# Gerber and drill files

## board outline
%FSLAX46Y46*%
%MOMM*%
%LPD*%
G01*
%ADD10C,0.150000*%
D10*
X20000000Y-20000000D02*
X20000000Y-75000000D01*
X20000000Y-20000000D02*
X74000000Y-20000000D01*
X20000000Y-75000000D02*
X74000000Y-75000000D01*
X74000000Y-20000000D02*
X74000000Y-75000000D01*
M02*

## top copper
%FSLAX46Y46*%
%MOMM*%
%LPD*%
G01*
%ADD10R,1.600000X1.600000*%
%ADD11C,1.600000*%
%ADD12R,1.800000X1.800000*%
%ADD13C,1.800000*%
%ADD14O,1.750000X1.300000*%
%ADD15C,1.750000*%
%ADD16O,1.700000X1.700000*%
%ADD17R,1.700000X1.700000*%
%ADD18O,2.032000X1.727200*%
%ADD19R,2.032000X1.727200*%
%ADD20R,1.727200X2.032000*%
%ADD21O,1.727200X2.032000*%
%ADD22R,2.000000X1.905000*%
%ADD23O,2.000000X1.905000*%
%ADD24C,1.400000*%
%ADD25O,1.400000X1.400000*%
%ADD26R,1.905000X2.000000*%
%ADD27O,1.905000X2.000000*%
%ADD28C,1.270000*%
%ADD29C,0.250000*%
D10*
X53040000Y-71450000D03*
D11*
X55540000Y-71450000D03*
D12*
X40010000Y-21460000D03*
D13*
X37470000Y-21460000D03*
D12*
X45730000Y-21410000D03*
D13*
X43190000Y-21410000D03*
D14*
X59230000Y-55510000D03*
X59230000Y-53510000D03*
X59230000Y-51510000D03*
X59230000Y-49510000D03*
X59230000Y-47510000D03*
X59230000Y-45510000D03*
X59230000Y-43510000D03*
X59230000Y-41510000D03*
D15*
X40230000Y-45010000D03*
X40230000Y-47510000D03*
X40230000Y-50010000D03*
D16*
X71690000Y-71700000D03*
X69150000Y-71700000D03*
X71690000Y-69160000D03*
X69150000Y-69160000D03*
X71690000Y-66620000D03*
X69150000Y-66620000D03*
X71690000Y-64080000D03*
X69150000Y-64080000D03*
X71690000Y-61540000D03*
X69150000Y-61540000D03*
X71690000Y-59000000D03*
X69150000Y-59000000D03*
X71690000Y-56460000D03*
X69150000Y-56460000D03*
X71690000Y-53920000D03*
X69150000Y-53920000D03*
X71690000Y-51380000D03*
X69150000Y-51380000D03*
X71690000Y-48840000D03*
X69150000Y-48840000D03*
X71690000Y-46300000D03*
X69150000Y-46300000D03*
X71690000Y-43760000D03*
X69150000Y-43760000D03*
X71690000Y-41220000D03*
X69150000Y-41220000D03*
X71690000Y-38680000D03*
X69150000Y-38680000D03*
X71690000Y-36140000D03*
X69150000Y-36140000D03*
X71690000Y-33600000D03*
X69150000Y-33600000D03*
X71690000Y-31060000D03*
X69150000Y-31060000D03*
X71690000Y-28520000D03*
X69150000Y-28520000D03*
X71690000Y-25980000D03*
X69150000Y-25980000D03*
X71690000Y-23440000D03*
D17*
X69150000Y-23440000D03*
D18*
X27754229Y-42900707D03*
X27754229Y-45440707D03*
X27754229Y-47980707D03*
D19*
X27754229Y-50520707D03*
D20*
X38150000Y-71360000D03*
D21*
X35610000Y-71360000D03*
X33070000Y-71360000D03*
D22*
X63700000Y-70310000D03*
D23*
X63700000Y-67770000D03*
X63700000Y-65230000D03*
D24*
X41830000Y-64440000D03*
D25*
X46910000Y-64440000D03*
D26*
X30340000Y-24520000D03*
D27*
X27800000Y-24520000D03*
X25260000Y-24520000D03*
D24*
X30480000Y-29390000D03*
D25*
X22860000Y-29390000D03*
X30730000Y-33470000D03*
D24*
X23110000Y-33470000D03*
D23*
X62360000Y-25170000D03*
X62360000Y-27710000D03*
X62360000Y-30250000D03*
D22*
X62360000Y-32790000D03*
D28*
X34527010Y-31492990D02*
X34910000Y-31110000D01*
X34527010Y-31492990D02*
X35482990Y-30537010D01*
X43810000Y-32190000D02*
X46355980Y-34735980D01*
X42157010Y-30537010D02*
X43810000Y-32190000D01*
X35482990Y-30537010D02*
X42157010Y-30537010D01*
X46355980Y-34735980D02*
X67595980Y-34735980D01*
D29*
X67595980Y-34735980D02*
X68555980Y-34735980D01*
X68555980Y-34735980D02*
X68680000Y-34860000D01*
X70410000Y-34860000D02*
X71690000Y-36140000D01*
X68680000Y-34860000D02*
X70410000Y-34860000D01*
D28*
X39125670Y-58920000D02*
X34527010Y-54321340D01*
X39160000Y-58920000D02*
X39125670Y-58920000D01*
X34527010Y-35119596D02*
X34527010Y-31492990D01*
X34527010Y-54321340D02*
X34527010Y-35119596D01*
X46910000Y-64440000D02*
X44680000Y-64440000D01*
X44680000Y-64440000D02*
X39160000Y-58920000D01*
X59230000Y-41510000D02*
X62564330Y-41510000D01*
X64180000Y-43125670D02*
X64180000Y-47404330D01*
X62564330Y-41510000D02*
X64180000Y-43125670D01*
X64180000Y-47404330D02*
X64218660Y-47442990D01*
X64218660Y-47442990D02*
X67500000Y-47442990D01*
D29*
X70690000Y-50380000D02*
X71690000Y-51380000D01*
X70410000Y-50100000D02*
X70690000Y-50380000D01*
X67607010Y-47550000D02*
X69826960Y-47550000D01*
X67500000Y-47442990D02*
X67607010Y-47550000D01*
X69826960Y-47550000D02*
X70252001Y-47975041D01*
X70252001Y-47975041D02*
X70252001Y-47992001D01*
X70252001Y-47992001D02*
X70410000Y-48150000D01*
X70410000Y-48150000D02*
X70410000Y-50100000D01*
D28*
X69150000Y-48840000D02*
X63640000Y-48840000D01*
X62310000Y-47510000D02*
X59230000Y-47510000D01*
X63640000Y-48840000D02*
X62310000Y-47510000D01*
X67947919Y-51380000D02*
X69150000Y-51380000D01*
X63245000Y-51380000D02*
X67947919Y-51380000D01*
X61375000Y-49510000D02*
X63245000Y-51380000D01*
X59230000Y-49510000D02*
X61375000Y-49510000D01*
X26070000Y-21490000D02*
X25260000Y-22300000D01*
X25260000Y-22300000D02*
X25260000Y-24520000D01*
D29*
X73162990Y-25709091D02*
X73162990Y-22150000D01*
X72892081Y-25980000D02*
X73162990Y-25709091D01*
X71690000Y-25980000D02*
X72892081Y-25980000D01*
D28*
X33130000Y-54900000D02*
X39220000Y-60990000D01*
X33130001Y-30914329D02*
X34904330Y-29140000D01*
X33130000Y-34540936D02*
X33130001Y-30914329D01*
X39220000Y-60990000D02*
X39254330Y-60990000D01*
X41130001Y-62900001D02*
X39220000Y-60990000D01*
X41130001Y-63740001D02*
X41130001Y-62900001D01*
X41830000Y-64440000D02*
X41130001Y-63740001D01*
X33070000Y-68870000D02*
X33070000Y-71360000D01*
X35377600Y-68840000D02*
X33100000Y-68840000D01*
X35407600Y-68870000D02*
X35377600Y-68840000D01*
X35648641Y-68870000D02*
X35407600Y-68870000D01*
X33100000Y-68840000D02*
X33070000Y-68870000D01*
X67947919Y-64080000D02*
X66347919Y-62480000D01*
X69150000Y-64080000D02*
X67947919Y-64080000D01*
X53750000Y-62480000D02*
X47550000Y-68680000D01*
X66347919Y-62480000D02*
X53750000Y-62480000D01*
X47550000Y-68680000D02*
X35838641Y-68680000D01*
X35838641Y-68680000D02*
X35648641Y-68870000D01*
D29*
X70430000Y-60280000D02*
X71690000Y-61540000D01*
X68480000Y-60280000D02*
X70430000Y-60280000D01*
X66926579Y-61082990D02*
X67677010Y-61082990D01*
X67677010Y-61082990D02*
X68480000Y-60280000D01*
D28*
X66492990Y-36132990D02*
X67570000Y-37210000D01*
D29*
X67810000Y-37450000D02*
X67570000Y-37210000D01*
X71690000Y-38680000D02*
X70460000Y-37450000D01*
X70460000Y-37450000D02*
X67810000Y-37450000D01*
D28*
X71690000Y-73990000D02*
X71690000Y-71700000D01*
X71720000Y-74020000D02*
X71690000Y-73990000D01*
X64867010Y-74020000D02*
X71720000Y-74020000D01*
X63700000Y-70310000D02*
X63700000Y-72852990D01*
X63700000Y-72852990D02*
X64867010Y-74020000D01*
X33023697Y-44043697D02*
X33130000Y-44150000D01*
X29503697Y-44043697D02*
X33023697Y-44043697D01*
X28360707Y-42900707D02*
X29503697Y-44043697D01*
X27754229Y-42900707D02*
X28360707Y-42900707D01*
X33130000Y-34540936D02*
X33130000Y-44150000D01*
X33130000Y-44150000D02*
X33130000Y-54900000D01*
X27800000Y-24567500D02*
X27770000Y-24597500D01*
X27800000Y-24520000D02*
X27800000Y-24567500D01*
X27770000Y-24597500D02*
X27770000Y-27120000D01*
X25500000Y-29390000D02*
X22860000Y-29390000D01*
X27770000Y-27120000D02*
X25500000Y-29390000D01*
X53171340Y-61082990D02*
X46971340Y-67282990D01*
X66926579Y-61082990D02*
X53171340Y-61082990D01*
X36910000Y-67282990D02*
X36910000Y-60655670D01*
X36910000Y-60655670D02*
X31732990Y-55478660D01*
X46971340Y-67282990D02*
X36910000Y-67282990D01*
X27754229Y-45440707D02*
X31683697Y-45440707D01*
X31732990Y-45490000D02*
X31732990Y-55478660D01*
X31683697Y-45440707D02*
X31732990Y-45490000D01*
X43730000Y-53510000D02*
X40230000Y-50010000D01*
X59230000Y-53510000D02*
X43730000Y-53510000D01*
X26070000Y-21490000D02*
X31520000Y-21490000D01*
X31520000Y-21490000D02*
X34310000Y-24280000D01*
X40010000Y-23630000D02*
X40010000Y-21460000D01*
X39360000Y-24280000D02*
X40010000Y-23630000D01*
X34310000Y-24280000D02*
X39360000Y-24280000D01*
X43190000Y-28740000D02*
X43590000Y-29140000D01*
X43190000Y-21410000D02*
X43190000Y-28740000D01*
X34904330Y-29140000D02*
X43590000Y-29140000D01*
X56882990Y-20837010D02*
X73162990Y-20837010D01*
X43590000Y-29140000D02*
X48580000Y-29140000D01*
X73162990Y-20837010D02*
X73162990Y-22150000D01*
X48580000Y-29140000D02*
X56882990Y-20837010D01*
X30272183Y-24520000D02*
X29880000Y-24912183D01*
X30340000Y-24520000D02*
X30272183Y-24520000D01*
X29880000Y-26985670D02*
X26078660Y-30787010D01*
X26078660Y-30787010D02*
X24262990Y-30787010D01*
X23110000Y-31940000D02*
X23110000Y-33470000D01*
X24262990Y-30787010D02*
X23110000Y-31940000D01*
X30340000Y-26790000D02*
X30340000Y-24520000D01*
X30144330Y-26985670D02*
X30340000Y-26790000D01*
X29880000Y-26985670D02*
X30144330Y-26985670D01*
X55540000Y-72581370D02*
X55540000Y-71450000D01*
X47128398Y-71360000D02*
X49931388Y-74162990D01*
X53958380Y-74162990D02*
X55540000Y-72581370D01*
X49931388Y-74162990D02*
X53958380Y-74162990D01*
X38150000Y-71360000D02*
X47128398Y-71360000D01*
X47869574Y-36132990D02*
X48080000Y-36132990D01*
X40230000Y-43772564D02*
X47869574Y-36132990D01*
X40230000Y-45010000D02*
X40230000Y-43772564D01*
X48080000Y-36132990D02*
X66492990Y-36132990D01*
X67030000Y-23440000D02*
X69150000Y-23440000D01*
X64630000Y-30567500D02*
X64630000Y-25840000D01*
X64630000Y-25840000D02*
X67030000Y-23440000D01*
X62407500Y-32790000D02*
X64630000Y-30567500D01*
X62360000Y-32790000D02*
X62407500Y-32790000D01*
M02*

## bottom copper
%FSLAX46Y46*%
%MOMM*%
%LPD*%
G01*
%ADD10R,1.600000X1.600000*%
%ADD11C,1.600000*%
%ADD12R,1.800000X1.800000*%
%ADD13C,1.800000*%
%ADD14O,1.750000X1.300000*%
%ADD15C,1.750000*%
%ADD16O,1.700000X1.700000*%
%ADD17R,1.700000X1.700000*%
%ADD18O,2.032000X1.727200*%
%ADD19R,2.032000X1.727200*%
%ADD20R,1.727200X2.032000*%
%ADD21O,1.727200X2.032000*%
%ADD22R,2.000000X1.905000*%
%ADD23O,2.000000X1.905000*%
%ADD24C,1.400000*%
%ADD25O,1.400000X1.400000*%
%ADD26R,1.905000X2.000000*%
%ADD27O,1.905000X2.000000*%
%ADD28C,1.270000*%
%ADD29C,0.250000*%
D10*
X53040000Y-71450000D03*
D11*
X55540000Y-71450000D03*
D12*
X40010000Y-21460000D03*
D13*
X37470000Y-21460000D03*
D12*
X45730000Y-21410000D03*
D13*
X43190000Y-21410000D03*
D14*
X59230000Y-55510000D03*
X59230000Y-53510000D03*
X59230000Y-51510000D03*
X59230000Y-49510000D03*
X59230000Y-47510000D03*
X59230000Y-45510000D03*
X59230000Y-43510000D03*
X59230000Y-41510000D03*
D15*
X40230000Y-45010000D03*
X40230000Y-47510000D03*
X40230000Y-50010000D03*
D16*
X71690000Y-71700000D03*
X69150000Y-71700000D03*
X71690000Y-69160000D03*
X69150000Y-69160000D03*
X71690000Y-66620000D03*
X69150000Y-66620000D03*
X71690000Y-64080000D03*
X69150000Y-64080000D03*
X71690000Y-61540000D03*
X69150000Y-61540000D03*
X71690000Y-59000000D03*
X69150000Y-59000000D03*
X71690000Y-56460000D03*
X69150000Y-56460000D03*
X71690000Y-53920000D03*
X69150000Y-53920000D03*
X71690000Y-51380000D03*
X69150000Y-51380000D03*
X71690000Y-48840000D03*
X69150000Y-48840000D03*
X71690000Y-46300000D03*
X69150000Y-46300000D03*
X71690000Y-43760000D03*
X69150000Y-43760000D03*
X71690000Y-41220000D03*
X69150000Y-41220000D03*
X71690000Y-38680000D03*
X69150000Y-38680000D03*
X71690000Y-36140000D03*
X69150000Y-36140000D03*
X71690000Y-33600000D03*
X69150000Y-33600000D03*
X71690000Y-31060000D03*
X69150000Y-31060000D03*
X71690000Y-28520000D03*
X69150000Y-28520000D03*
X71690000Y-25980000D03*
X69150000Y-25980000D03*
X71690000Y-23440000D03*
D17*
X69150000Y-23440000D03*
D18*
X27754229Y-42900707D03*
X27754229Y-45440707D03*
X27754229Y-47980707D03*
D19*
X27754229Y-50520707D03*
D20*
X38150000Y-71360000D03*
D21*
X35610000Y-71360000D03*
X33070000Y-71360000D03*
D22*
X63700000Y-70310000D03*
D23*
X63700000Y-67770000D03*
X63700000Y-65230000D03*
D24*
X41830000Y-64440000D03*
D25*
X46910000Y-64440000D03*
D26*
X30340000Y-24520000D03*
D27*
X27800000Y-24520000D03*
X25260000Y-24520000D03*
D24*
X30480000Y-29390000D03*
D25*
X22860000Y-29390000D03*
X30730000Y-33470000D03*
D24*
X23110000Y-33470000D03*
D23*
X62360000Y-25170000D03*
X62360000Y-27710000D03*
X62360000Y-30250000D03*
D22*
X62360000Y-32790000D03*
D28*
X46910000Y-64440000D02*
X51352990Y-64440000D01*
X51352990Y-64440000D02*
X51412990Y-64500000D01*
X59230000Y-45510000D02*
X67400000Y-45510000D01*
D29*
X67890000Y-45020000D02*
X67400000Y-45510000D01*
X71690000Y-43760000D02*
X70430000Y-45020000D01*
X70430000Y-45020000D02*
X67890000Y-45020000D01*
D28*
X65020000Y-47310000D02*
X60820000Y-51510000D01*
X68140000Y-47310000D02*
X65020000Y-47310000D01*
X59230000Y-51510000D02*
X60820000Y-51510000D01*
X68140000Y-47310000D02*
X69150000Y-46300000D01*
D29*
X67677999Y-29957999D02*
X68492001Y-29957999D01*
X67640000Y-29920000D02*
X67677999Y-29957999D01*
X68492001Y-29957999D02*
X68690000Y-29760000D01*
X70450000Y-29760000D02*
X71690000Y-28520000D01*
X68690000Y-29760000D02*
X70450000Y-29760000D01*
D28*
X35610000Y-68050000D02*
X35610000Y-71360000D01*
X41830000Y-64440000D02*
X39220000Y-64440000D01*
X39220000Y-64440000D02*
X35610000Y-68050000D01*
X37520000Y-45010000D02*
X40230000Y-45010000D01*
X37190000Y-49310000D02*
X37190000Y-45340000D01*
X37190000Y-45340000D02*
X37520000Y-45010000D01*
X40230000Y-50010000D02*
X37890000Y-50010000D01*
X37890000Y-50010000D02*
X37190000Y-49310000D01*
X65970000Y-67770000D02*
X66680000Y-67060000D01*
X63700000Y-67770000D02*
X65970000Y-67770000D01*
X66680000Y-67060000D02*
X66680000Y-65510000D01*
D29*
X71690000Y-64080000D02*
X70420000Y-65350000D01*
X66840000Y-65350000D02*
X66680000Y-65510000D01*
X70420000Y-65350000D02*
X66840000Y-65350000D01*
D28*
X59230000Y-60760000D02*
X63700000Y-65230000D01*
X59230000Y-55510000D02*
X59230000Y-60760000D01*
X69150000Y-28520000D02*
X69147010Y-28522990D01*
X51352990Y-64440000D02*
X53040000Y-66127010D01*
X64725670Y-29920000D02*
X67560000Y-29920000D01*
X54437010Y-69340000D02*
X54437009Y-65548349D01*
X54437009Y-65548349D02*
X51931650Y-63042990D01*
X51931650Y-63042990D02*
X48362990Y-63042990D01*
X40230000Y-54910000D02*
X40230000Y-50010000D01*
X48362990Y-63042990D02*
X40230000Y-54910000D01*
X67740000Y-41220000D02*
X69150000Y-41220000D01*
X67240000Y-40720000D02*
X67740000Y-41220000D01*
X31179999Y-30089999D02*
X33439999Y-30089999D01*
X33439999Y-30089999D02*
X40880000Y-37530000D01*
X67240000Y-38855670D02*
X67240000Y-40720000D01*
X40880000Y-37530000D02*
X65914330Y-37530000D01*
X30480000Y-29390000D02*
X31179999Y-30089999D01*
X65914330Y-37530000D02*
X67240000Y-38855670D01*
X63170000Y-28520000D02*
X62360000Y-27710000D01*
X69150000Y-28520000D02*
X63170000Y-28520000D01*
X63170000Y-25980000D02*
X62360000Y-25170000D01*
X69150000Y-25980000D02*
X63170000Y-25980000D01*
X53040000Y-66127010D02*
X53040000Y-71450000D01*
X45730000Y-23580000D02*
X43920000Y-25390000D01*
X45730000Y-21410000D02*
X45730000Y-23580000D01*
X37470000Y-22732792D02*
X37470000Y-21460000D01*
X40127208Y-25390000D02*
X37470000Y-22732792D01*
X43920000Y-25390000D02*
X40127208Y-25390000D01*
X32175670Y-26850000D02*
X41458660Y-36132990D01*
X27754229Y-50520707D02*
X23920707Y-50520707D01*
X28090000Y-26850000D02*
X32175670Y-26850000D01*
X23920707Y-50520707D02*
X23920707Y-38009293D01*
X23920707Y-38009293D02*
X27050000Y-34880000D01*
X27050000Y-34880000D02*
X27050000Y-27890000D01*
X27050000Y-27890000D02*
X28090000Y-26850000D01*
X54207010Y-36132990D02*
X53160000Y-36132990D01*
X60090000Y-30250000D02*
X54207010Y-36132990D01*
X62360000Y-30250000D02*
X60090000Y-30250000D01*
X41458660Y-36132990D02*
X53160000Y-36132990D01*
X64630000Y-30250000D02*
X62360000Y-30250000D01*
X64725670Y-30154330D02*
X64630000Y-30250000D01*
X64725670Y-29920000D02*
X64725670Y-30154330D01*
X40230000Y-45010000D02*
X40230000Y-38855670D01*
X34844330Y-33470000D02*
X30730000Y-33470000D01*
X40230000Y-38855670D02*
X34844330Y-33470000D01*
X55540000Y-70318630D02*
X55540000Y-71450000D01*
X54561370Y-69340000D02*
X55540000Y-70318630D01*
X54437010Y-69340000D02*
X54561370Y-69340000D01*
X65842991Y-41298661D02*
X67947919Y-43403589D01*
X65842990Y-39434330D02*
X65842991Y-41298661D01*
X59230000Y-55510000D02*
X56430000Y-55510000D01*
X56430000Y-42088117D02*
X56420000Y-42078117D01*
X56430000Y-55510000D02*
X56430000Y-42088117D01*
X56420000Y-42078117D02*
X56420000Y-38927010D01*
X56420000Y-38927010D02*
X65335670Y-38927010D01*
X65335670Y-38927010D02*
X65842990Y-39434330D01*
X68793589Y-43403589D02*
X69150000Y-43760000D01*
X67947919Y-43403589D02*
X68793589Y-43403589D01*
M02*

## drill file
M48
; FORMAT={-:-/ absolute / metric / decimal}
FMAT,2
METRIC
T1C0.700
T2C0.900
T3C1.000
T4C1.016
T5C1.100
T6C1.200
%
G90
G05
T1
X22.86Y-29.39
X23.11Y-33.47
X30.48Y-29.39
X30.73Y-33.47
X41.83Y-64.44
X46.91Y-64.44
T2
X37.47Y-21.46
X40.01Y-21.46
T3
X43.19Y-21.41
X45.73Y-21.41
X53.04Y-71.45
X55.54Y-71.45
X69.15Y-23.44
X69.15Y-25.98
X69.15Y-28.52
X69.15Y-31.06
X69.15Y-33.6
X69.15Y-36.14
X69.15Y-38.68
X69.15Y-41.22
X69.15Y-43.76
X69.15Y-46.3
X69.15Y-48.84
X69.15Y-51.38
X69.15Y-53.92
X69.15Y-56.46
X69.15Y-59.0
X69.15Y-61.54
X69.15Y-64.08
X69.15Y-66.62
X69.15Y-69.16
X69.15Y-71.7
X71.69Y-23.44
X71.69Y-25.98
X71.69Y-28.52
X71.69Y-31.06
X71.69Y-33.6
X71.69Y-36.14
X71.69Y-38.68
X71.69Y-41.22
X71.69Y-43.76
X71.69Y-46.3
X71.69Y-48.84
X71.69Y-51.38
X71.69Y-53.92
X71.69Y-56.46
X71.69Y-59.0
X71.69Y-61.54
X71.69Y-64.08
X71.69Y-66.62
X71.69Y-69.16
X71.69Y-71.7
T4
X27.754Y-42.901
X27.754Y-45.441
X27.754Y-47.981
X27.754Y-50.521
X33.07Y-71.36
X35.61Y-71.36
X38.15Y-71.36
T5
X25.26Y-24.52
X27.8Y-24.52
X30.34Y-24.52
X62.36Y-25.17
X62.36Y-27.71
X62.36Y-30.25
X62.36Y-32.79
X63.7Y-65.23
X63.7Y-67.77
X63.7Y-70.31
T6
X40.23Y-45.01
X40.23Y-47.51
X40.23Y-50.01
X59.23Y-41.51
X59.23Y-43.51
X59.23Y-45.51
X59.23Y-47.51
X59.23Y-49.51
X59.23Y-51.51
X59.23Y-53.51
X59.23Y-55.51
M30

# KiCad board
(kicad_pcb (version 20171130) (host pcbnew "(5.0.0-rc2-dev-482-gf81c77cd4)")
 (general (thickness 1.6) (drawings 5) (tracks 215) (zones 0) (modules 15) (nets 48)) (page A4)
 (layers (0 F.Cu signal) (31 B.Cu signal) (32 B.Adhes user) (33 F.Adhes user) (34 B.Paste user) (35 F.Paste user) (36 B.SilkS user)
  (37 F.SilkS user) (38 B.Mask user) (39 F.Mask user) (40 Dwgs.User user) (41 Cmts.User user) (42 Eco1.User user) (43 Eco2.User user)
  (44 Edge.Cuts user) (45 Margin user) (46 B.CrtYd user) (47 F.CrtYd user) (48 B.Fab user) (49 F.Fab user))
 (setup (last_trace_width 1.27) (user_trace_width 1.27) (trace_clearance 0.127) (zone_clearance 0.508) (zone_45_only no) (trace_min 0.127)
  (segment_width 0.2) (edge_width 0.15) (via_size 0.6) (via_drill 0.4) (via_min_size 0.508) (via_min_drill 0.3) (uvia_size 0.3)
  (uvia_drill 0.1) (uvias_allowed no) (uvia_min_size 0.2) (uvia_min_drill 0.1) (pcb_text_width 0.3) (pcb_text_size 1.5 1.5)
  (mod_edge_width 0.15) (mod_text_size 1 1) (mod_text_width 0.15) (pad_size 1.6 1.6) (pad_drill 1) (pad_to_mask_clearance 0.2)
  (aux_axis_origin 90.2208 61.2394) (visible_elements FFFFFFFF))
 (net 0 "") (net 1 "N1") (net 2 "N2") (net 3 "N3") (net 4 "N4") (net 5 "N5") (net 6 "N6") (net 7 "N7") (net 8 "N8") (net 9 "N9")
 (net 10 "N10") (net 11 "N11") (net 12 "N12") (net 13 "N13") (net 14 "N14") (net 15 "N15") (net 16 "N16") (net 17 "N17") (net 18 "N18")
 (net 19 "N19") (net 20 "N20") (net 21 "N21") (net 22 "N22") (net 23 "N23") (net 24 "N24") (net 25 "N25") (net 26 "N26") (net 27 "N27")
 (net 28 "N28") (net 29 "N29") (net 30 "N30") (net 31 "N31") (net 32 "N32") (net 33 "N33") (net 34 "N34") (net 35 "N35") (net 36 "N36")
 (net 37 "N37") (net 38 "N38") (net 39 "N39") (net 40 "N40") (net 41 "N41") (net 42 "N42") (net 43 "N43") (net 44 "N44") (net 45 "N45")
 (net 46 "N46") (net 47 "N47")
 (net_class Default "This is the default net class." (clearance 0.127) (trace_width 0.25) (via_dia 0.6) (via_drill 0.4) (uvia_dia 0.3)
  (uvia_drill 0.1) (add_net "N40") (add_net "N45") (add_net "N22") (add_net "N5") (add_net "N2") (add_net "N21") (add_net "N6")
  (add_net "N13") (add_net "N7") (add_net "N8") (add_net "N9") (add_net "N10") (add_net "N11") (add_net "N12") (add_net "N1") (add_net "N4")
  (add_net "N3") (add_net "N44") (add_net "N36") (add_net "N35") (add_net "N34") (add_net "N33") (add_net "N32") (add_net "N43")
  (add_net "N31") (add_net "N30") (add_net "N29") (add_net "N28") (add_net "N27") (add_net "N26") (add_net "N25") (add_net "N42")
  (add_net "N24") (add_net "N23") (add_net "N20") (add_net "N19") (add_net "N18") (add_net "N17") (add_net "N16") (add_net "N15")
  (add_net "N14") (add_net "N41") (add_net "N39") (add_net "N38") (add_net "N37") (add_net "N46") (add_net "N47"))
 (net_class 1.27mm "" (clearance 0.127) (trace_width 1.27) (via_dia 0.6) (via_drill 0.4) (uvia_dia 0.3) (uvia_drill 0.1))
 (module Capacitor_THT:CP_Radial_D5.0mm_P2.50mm (layer F.Cu) (at 53.04 71.45)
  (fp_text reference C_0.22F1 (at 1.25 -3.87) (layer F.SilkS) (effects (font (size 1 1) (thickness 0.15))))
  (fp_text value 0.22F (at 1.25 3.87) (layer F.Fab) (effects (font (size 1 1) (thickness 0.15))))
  (pad 1 thru_hole rect (at 0 0) (size 1.6 1.6) (drill 1) (layers *.Cu *.Mask) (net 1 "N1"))
  (pad 2 thru_hole circle (at 2.5 0) (size 1.6 1.6) (drill 1) (layers *.Cu *.Mask) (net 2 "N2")))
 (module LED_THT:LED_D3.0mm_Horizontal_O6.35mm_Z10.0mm (layer F.Cu) (at 40.01 21.46 180)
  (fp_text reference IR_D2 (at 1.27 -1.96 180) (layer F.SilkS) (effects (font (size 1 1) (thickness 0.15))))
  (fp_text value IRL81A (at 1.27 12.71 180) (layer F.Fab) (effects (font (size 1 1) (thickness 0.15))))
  (pad 1 thru_hole rect (at 0 0 180) (size 1.8 1.8) (drill 0.9) (layers *.Cu *.Mask) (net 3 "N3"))
  (pad 2 thru_hole circle (at 2.54 0 180) (size 1.8 1.8) (drill 0.9) (layers *.Cu *.Mask) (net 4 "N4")))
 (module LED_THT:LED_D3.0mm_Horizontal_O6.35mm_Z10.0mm (layer F.Cu) (at 45.73 21.41 180)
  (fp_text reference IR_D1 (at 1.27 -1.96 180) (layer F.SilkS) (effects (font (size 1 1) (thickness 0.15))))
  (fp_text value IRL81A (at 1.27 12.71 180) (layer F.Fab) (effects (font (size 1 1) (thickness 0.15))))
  (pad 1 thru_hole rect (at 0 0 180) (size 1.8 1.8) (drill 1) (layers *.Cu *.Mask) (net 4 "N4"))
  (pad 2 thru_hole circle (at 2.54 0 180) (size 1.8 1.8) (drill 1) (layers *.Cu *.Mask) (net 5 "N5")))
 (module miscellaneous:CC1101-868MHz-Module (layer F.Cu) (at 49.73 48.51 180)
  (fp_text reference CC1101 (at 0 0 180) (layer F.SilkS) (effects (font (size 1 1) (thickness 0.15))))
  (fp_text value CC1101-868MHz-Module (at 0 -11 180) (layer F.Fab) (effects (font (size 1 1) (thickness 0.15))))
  (pad 1 thru_hole oval (at -9.5 -7 180) (size 1.75 1.3) (drill 1.2) (layers *.Cu *.Mask) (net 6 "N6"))
  (pad 2 thru_hole oval (at -9.5 -5 180) (size 1.75 1.3) (drill 1.2) (layers *.Cu *.Mask) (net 2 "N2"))
  (pad 3 thru_hole oval (at -9.5 -3 180) (size 1.75 1.3) (drill 1.2) (layers *.Cu *.Mask) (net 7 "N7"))
  (pad 4 thru_hole oval (at -9.5 -1 180) (size 1.75 1.3) (drill 1.2) (layers *.Cu *.Mask) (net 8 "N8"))
  (pad 5 thru_hole oval (at -9.5 1 180) (size 1.75 1.3) (drill 1.2) (layers *.Cu *.Mask) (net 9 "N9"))
  (pad 6 thru_hole oval (at -9.5 3 180) (size 1.75 1.3) (drill 1.2) (layers *.Cu *.Mask) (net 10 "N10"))
  (pad 7 thru_hole oval (at -9.5 5 180) (size 1.75 1.3) (drill 1.2) (layers *.Cu *.Mask) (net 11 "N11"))
  (pad 8 thru_hole oval (at -9.5 7 180) (size 1.75 1.3) (drill 1.2) (layers *.Cu *.Mask) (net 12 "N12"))
  (pad 9 thru_hole circle (at 9.5 3.5 180) (size 1.75 1.75) (drill 1.2) (layers *.Cu *.Mask) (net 2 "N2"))
  (pad 10 thru_hole circle (at 9.5 1 180) (size 1.75 1.75) (drill 1.2) (layers *.Cu *.Mask) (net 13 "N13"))
  (pad 11 thru_hole circle (at 9.5 -1.5 180) (size 1.75 1.75) (drill 1.2) (layers *.Cu *.Mask) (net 2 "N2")))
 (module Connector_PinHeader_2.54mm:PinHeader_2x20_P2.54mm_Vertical (layer F.Cu) (at 69.15 23.44)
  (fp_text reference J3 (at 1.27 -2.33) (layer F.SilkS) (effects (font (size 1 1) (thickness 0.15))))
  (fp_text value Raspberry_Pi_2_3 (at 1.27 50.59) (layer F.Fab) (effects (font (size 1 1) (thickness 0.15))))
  (pad 40 thru_hole oval (at 2.54 48.26) (size 1.7 1.7) (drill 1) (layers *.Cu *.Mask) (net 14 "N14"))
  (pad 39 thru_hole oval (at 0 48.26) (size 1.7 1.7) (drill 1) (layers *.Cu *.Mask) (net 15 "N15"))
  (pad 38 thru_hole oval (at 2.54 45.72) (size 1.7 1.7) (drill 1) (layers *.Cu *.Mask) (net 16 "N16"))
  (pad 37 thru_hole oval (at 0 45.72) (size 1.7 1.7) (drill 1) (layers *.Cu *.Mask) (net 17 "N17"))
  (pad 36 thru_hole oval (at 2.54 43.18) (size 1.7 1.7) (drill 1) (layers *.Cu *.Mask) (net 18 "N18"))
  (pad 35 thru_hole oval (at 0 43.18) (size 1.7 1.7) (drill 1) (layers *.Cu *.Mask) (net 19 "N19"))
  (pad 34 thru_hole oval (at 2.54 40.64) (size 1.7 1.7) (drill 1) (layers *.Cu *.Mask) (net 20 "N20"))
  (pad 33 thru_hole oval (at 0 40.64) (size 1.7 1.7) (drill 1) (layers *.Cu *.Mask) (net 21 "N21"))
  (pad 32 thru_hole oval (at 2.54 38.1) (size 1.7 1.7) (drill 1) (layers *.Cu *.Mask) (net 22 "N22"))
  (pad 31 thru_hole oval (at 0 38.1) (size 1.7 1.7) (drill 1) (layers *.Cu *.Mask) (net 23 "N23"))
  (pad 30 thru_hole oval (at 2.54 35.56) (size 1.7 1.7) (drill 1) (layers *.Cu *.Mask) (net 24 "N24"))
  (pad 29 thru_hole oval (at 0 35.56) (size 1.7 1.7) (drill 1) (layers *.Cu *.Mask) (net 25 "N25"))
  (pad 28 thru_hole oval (at 2.54 33.02) (size 1.7 1.7) (drill 1) (layers *.Cu *.Mask) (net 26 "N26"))
  (pad 27 thru_hole oval (at 0 33.02) (size 1.7 1.7) (drill 1) (layers *.Cu *.Mask) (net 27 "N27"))
  (pad 26 thru_hole oval (at 2.54 30.48) (size 1.7 1.7) (drill 1) (layers *.Cu *.Mask) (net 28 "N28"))
  (pad 25 thru_hole oval (at 0 30.48) (size 1.7 1.7) (drill 1) (layers *.Cu *.Mask) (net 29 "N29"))
  (pad 24 thru_hole oval (at 2.54 27.94) (size 1.7 1.7) (drill 1) (layers *.Cu *.Mask) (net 12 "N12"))
  (pad 23 thru_hole oval (at 0 27.94) (size 1.7 1.7) (drill 1) (layers *.Cu *.Mask) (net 8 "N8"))
  (pad 22 thru_hole oval (at 2.54 25.4) (size 1.7 1.7) (drill 1) (layers *.Cu *.Mask) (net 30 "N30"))
  (pad 21 thru_hole oval (at 0 25.4) (size 1.7 1.7) (drill 1) (layers *.Cu *.Mask) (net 9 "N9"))
  (pad 20 thru_hole oval (at 2.54 22.86) (size 1.7 1.7) (drill 1) (layers *.Cu *.Mask) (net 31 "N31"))
  (pad 19 thru_hole oval (at 0 22.86) (size 1.7 1.7) (drill 1) (layers *.Cu *.Mask) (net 7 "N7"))
  (pad 18 thru_hole oval (at 2.54 20.32) (size 1.7 1.7) (drill 1) (layers *.Cu *.Mask) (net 10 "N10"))
  (pad 17 thru_hole oval (at 0 20.32) (size 1.7 1.7) (drill 1) (layers *.Cu *.Mask) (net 6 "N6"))
  (pad 16 thru_hole oval (at 2.54 17.78) (size 1.7 1.7) (drill 1) (layers *.Cu *.Mask) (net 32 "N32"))
  (pad 15 thru_hole oval (at 0 17.78) (size 1.7 1.7) (drill 1) (layers *.Cu *.Mask) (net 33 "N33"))
  (pad 14 thru_hole oval (at 2.54 15.24) (size 1.7 1.7) (drill 1) (layers *.Cu *.Mask) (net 2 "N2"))
  (pad 13 thru_hole oval (at 0 15.24) (size 1.7 1.7) (drill 1) (layers *.Cu *.Mask) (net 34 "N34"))
  (pad 12 thru_hole oval (at 2.54 12.7) (size 1.7 1.7) (drill 1) (layers *.Cu *.Mask) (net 1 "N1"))
  (pad 11 thru_hole oval (at 0 12.7) (size 1.7 1.7) (drill 1) (layers *.Cu *.Mask) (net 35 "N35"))
  (pad 10 thru_hole oval (at 2.54 10.16) (size 1.7 1.7) (drill 1) (layers *.Cu *.Mask) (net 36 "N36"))
  (pad 9 thru_hole oval (at 0 10.16) (size 1.7 1.7) (drill 1) (layers *.Cu *.Mask) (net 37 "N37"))
  (pad 8 thru_hole oval (at 2.54 7.62) (size 1.7 1.7) (drill 1) (layers *.Cu *.Mask) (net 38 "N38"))
  (pad 7 thru_hole oval (at 0 7.62) (size 1.7 1.7) (drill 1) (layers *.Cu *.Mask) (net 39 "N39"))
  (pad 6 thru_hole oval (at 2.54 5.08) (size 1.7 1.7) (drill 1) (layers *.Cu *.Mask) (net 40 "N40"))
  (pad 5 thru_hole oval (at 0 5.08) (size 1.7 1.7) (drill 1) (layers *.Cu *.Mask) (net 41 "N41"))
  (pad 4 thru_hole oval (at 2.54 2.54) (size 1.7 1.7) (drill 1) (layers *.Cu *.Mask) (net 5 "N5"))
  (pad 3 thru_hole oval (at 0 2.54) (size 1.7 1.7) (drill 1) (layers *.Cu *.Mask) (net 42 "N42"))
  (pad 2 thru_hole oval (at 2.54 0) (size 1.7 1.7) (drill 1) (layers *.Cu *.Mask) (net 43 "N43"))
  (pad 1 thru_hole rect (at 0 0) (size 1.7 1.7) (drill 1) (layers *.Cu *.Mask) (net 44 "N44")))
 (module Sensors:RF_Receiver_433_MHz (layer F.Cu) (at 27.73 45.46 90)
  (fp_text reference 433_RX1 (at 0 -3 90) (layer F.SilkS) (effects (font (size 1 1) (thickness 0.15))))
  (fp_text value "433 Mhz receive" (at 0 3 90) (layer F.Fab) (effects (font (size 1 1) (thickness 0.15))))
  (pad 4 thru_hole oval (at 2.559293 0.024229 180) (size 2.032 1.7272) (drill 1.016) (layers *.Cu *.Mask F.SilkS) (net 5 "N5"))
  (pad 3 thru_hole oval (at 0.019293 0.024229 180) (size 2.032 1.7272) (drill 1.016) (layers *.Cu *.Mask F.SilkS) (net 22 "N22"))
  (pad 2 thru_hole oval (at -2.520707 0.024229 180) (size 2.032 1.7272) (drill 1.016) (layers *.Cu *.Mask F.SilkS) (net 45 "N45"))
  (pad 1 thru_hole rect (at -5.060707 0.024229 180) (size 2.032 1.7272) (drill 1.016) (layers *.Cu *.Mask F.SilkS) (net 40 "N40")))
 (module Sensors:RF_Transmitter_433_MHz (layer F.Cu) (at 35.61 71.36 180)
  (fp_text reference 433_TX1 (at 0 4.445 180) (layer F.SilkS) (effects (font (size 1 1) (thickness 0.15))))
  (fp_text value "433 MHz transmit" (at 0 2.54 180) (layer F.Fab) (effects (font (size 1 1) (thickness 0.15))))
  (pad 1 thru_hole rect (at -2.54 0 270) (size 2.032 1.7272) (drill 1.016) (layers *.Cu *.Mask F.SilkS) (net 2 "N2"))
  (pad 2 thru_hole oval (at 0 0 270) (size 2.032 1.7272) (drill 1.016) (layers *.Cu *.Mask F.SilkS) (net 5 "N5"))
  (pad 3 thru_hole oval (at 2.54 0 270) (size 2.032 1.7272) (drill 1.016) (layers *.Cu *.Mask F.SilkS) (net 21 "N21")))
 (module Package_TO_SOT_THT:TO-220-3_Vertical (layer F.Cu) (at 63.7 70.31 90)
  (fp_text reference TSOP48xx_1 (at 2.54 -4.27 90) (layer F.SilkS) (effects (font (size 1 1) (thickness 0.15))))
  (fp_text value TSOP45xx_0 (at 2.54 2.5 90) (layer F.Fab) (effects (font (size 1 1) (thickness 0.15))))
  (pad 1 thru_hole rect (at 0 0 90) (size 1.905 2) (drill 1.1) (layers *.Cu *.Mask) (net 14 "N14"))
  (pad 2 thru_hole oval (at 2.54 0 90) (size 1.905 2) (drill 1.1) (layers *.Cu *.Mask) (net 20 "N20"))
  (pad 3 thru_hole oval (at 5.08 0 90) (size 1.905 2) (drill 1.1) (layers *.Cu *.Mask) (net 6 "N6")))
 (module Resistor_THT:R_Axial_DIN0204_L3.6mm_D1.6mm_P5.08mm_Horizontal (layer F.Cu) (at 41.83 64.44)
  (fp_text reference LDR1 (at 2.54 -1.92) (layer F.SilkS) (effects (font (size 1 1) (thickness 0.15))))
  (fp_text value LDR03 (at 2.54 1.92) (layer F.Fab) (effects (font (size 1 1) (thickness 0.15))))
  (pad 1 thru_hole circle (at 0 0) (size 1.4 1.4) (drill 0.7) (layers *.Cu *.Mask) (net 5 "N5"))
  (pad 2 thru_hole oval (at 5.08 0) (size 1.4 1.4) (drill 0.7) (layers *.Cu *.Mask) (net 1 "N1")))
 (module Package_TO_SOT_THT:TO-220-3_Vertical (layer F.Cu) (at 30.34 24.52 180)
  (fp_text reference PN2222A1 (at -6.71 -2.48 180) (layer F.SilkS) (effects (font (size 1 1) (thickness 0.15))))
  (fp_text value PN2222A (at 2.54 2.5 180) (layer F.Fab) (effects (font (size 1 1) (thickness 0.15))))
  (pad 1 thru_hole rect (at 0 0 180) (size 1.905 2) (drill 1.1) (layers *.Cu *.Mask) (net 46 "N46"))
  (pad 2 thru_hole oval (at 2.54 0 180) (size 1.905 2) (drill 1.1) (layers *.Cu *.Mask) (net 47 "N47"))
  (pad 3 thru_hole oval (at 5.08 0 180) (size 1.905 2) (drill 1.1) (layers *.Cu *.Mask) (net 3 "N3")))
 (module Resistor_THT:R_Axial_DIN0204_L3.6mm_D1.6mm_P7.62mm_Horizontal (layer F.Cu) (at 30.48 29.39 180)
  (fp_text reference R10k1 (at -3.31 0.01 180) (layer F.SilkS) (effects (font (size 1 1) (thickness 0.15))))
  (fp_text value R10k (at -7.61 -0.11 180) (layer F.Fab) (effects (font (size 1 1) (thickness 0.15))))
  (pad 1 thru_hole circle (at 0 0 180) (size 1.4 1.4) (drill 0.7) (layers *.Cu *.Mask) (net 33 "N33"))
  (pad 2 thru_hole oval (at 7.62 0 180) (size 1.4 1.4) (drill 0.7) (layers *.Cu *.Mask) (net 47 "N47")))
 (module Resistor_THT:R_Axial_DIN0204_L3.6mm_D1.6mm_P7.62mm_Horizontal (layer F.Cu) (at 23.11 33.47)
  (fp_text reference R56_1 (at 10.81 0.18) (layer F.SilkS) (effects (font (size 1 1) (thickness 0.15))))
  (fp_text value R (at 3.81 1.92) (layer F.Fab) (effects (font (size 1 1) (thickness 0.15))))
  (pad 2 thru_hole oval (at 7.62 0) (size 1.4 1.4) (drill 0.7) (layers *.Cu *.Mask) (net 2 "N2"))
  (pad 1 thru_hole circle (at 0 0) (size 1.4 1.4) (drill 0.7) (layers *.Cu *.Mask) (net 46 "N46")))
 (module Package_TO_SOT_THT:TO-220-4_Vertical (layer F.Cu) (at 62.36 32.79 90)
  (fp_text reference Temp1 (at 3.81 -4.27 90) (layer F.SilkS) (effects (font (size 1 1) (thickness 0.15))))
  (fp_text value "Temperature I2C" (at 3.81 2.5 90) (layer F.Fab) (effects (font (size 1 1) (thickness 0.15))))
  (pad 4 thru_hole oval (at 7.62 0 90) (size 1.905 2) (drill 1.1) (layers *.Cu *.Mask) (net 42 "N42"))
  (pad 3 thru_hole oval (at 5.08 0 90) (size 1.905 2) (drill 1.1) (layers *.Cu *.Mask) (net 41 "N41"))
  (pad 2 thru_hole oval (at 2.54 0 90) (size 1.905 2) (drill 1.1) (layers *.Cu *.Mask) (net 40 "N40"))
  (pad 1 thru_hole rect (at 0 0 90) (size 1.905 2) (drill 1.1) (layers *.Cu *.Mask) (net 44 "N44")))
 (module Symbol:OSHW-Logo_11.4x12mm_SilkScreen (layer F.Cu) (at 51.43 27.68)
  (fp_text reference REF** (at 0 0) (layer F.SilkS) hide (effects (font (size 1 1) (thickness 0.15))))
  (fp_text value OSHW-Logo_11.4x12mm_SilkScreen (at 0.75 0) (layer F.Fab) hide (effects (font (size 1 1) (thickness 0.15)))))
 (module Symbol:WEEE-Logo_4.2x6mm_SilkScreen (layer F.Cu) (at 22.62 71.55)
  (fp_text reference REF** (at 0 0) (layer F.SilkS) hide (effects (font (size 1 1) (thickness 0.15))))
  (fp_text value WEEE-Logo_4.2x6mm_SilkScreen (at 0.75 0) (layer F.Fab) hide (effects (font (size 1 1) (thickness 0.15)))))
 (gr_line (start 20 20) (end 20 75) (angle 90) (layer Edge.Cuts) (width 0.15))
 (gr_line (start 20 20) (end 74 20) (angle 90) (layer Edge.Cuts) (width 0.15))
 (gr_line (start 20 75) (end 74 75) (angle 90) (layer Edge.Cuts) (width 0.15))
 (gr_line (start 74 20) (end 74 75) (angle 90) (layer Edge.Cuts) (width 0.15))
 (segment (start 34.52701 31.49299) (end 34.91 31.11) (width 1.27) (layer F.Cu) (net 1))
 (segment (start 34.52701 31.49299) (end 35.48299 30.53701) (width 1.27) (layer F.Cu) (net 1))
 (segment (start 43.81 32.19) (end 46.35598 34.73598) (width 1.27) (layer F.Cu) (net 1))
 (segment (start 42.15701 30.53701) (end 43.81 32.19) (width 1.27) (layer F.Cu) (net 1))
 (segment (start 35.48299 30.53701) (end 42.15701 30.53701) (width 1.27) (layer F.Cu) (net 1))
 (segment (start 46.35598 34.73598) (end 67.59598 34.73598) (width 1.27) (layer F.Cu) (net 1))
 (segment (start 67.59598 34.73598) (end 68.55598 34.73598) (width 0.25) (layer F.Cu) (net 1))
 (segment (start 68.55598 34.73598) (end 68.68 34.86) (width 0.25) (layer F.Cu) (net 1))
 (segment (start 70.41 34.86) (end 71.69 36.14) (width 0.25) (layer F.Cu) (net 1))
 (segment (start 68.68 34.86) (end 70.41 34.86) (width 0.25) (layer F.Cu) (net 1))
 (segment (start 39.12567 58.92) (end 34.52701 54.32134) (width 1.27) (layer F.Cu) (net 1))
 (segment (start 39.16 58.92) (end 39.12567 58.92) (width 1.27) (layer F.Cu) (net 1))
 (segment (start 34.52701 35.119596) (end 34.52701 31.49299) (width 1.27) (layer F.Cu) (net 1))
 (segment (start 34.52701 54.32134) (end 34.52701 35.119596) (width 1.27) (layer F.Cu) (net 1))
 (segment (start 46.91 64.44) (end 44.68 64.44) (width 1.27) (layer F.Cu) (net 1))
 (segment (start 44.68 64.44) (end 39.16 58.92) (width 1.27) (layer F.Cu) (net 1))
 (segment (start 46.91 64.44) (end 51.35299 64.44) (width 1.27) (layer B.Cu) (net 1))
 (segment (start 51.35299 64.44) (end 51.41299 64.5) (width 1.27) (layer B.Cu) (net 1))
 (segment (start 59.23 41.51) (end 62.56433 41.51) (width 1.27) (layer F.Cu) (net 12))
 (segment (start 64.18 43.12567) (end 64.18 47.40433) (width 1.27) (layer F.Cu) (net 12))
 (segment (start 62.56433 41.51) (end 64.18 43.12567) (width 1.27) (layer F.Cu) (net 12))
 (segment (start 64.18 47.40433) (end 64.21866 47.44299) (width 1.27) (layer F.Cu) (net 12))
 (segment (start 64.21866 47.44299) (end 67.5 47.44299) (width 1.27) (layer F.Cu) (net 12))
 (segment (start 70.69 50.38) (end 71.69 51.38) (width 0.25) (layer F.Cu) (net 12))
 (segment (start 70.41 50.1) (end 70.69 50.38) (width 0.25) (layer F.Cu) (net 12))
 (segment (start 67.60701 47.55) (end 69.82696 47.55) (width 0.25) (layer F.Cu) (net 12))
 (segment (start 67.5 47.44299) (end 67.60701 47.55) (width 0.25) (layer F.Cu) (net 12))
 (segment (start 69.82696 47.55) (end 70.252001 47.975041) (width 0.25) (layer F.Cu) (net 12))
 (segment (start 70.252001 47.975041) (end 70.252001 47.992001) (width 0.25) (layer F.Cu) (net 12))
 (segment (start 70.252001 47.992001) (end 70.41 48.15) (width 0.25) (layer F.Cu) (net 12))
 (segment (start 70.41 48.15) (end 70.41 50.1) (width 0.25) (layer F.Cu) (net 12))
 (segment (start 59.23 45.51) (end 67.4 45.51) (width 1.27) (layer B.Cu) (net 10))
 (segment (start 67.89 45.02) (end 67.4 45.51) (width 0.25) (layer B.Cu) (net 10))
 (segment (start 71.69 43.76) (end 70.43 45.02) (width 0.25) (layer B.Cu) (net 10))
 (segment (start 70.43 45.02) (end 67.89 45.02) (width 0.25) (layer B.Cu) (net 10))
 (segment (start 69.15 48.84) (end 63.64 48.84) (width 1.27) (layer F.Cu) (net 9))
 (segment (start 62.31 47.51) (end 59.23 47.51) (width 1.27) (layer F.Cu) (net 9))
 (segment (start 63.64 48.84) (end 62.31 47.51) (width 1.27) (layer F.Cu) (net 9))
 (segment (start 67.947919 51.38) (end 69.15 51.38) (width 1.27) (layer F.Cu) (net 8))
 (segment (start 63.245 51.38) (end 67.947919 51.38) (width 1.27) (layer F.Cu) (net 8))
 (segment (start 61.375 49.51) (end 63.245 51.38) (width 1.27) (layer F.Cu) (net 8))
 (segment (start 59.23 49.51) (end 61.375 49.51) (width 1.27) (layer F.Cu) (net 8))
 (segment (start 65.02 47.31) (end 60.82 51.51) (width 1.27) (layer B.Cu) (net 7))
 (segment (start 68.14 47.31) (end 65.02 47.31) (width 1.27) (layer B.Cu) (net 7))
 (segment (start 59.23 51.51) (end 60.82 51.51) (width 1.27) (layer B.Cu) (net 7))
 (segment (start 68.14 47.31) (end 69.15 46.3) (width 1.27) (layer B.Cu) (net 7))
 (segment (start 26.07 21.49) (end 25.26 22.3) (width 1.27) (layer F.Cu) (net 3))
 (segment (start 25.26 22.3) (end 25.26 24.52) (width 1.27) (layer F.Cu) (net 3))
 (segment (start 67.677999 29.957999) (end 68.492001 29.957999) (width 0.25) (layer B.Cu) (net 40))
 (segment (start 67.64 29.92) (end 67.677999 29.957999) (width 0.25) (layer B.Cu) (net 40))
 (segment (start 68.492001 29.957999) (end 68.69 29.76) (width 0.25) (layer B.Cu) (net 40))
 (segment (start 70.45 29.76) (end 71.69 28.52) (width 0.25) (layer B.Cu) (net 40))
 (segment (start 68.69 29.76) (end 70.45 29.76) (width 0.25) (layer B.Cu) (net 40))
 (segment (start 73.16299 25.709091) (end 73.16299 22.15) (width 0.25) (layer F.Cu) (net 5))
 (segment (start 72.892081 25.98) (end 73.16299 25.709091) (width 0.25) (layer F.Cu) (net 5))
 (segment (start 71.69 25.98) (end 72.892081 25.98) (width 0.25) (layer F.Cu) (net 5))
 (segment (start 33.13 54.9) (end 39.22 60.99) (width 1.27) (layer F.Cu) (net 5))
 (segment (start 33.130001 30.914329) (end 34.90433 29.14) (width 1.27) (layer F.Cu) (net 5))
 (segment (start 33.13 34.540936) (end 33.130001 30.914329) (width 1.27) (layer F.Cu) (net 5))
 (segment (start 39.22 60.99) (end 39.25433 60.99) (width 1.27) (layer F.Cu) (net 5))
 (segment (start 41.130001 62.900001) (end 39.22 60.99) (width 1.27) (layer F.Cu) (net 5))
 (segment (start 41.130001 63.740001) (end 41.130001 62.900001) (width 1.27) (layer F.Cu) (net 5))
 (segment (start 41.83 64.44) (end 41.130001 63.740001) (width 1.27) (layer F.Cu) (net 5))
 (segment (start 35.61 68.05) (end 35.61 71.36) (width 1.27) (layer B.Cu) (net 5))
 (segment (start 41.83 64.44) (end 39.22 64.44) (width 1.27) (layer B.Cu) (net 5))
 (segment (start 39.22 64.44) (end 35.61 68.05) (width 1.27) (layer B.Cu) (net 5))
 (segment (start 33.07 68.87) (end 33.07 71.36) (width 1.27) (layer F.Cu) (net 21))
 (segment (start 35.3776 68.84) (end 33.1 68.84) (width 1.27) (layer F.Cu) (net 21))
 (segment (start 35.4076 68.87) (end 35.3776 68.84) (width 1.27) (layer F.Cu) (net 21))
 (segment (start 35.648641 68.87) (end 35.4076 68.87) (width 1.27) (layer F.Cu) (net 21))
 (segment (start 33.1 68.84) (end 33.07 68.87) (width 1.27) (layer F.Cu) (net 21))
 (segment (start 67.947919 64.08) (end 66.347919 62.48) (width 1.27) (layer F.Cu) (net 21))
 (segment (start 69.15 64.08) (end 67.947919 64.08) (width 1.27) (layer F.Cu) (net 21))
 (segment (start 53.75 62.48) (end 47.55 68.68) (width 1.27) (layer F.Cu) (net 21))
 (segment (start 66.347919 62.48) (end 53.75 62.48) (width 1.27) (layer F.Cu) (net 21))
 (segment (start 47.55 68.68) (end 35.838641 68.68) (width 1.27) (layer F.Cu) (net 21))
 (segment (start 35.838641 68.68) (end 35.648641 68.87) (width 1.27) (layer F.Cu) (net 21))
 (segment (start 70.43 60.28) (end 71.69 61.54) (width 0.25) (layer F.Cu) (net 22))
 (segment (start 68.48 60.28) (end 70.43 60.28) (width 0.25) (layer F.Cu) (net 22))
 (segment (start 66.926579 61.08299) (end 67.67701 61.08299) (width 0.25) (layer F.Cu) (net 22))
 (segment (start 67.67701 61.08299) (end 68.48 60.28) (width 0.25) (layer F.Cu) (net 22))
 (segment (start 66.49299 36.13299) (end 67.57 37.21) (width 1.27) (layer F.Cu) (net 2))
 (segment (start 67.81 37.45) (end 67.57 37.21) (width 0.25) (layer F.Cu) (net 2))
 (segment (start 71.69 38.68) (end 70.46 37.45) (width 0.25) (layer F.Cu) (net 2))
 (segment (start 70.46 37.45) (end 67.81 37.45) (width 0.25) (layer F.Cu) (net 2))
 (segment (start 37.52 45.01) (end 40.23 45.01) (width 1.27) (layer B.Cu) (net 2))
 (segment (start 37.19 49.31) (end 37.19 45.34) (width 1.27) (layer B.Cu) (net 2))
 (segment (start 37.19 45.34) (end 37.52 45.01) (width 1.27) (layer B.Cu) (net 2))
 (segment (start 40.23 50.01) (end 37.89 50.01) (width 1.27) (layer B.Cu) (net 2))
 (segment (start 37.89 50.01) (end 37.19 49.31) (width 1.27) (layer B.Cu) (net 2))
 (segment (start 71.69 73.99) (end 71.69 71.7) (width 1.27) (layer F.Cu) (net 14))
 (segment (start 71.72 74.02) (end 71.69 73.99) (width 1.27) (layer F.Cu) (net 14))
 (segment (start 64.86701 74.02) (end 71.72 74.02) (width 1.27) (layer F.Cu) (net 14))
 (segment (start 63.7 70.31) (end 63.7 72.85299) (width 1.27) (layer F.Cu) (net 14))
 (segment (start 63.7 72.85299) (end 64.86701 74.02) (width 1.27) (layer F.Cu) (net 14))
 (segment (start 65.97 67.77) (end 66.68 67.06) (width 1.27) (layer B.Cu) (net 20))
 (segment (start 63.7 67.77) (end 65.97 67.77) (width 1.27) (layer B.Cu) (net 20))
 (segment (start 66.68 67.06) (end 66.68 65.51) (width 1.27) (layer B.Cu) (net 20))
 (segment (start 71.69 64.08) (end 70.42 65.35) (width 0.25) (layer B.Cu) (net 20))
 (segment (start 66.84 65.35) (end 66.68 65.51) (width 0.25) (layer B.Cu) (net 20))
 (segment (start 70.42 65.35) (end 66.84 65.35) (width 0.25) (layer B.Cu) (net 20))
 (segment (start 59.23 60.76) (end 63.7 65.23) (width 1.27) (layer B.Cu) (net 6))
 (segment (start 59.23 55.51) (end 59.23 60.76) (width 1.27) (layer B.Cu) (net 6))
 (segment (start 69.15 28.52) (end 69.14701 28.52299) (width 1.27) (layer B.Cu) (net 41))
 (segment (start 51.35299 64.44) (end 53.04 66.12701) (width 1.27) (layer B.Cu) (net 1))
 (segment (start 64.72567 29.92) (end 67.56 29.92) (width 1.27) (layer B.Cu) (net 40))
 (segment (start 33.023697 44.043697) (end 33.13 44.15) (width 1.27) (layer F.Cu) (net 5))
 (segment (start 29.503697 44.043697) (end 33.023697 44.043697) (width 1.27) (layer F.Cu) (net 5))
 (segment (start 28.360707 42.900707) (end 29.503697 44.043697) (width 1.27) (layer F.Cu) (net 5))
 (segment (start 27.754229 42.900707) (end 28.360707 42.900707) (width 1.27) (layer F.Cu) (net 5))
 (segment (start 33.13 34.540936) (end 33.13 44.15) (width 1.27) (layer F.Cu) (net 5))
 (segment (start 33.13 44.15) (end 33.13 54.9) (width 1.27) (layer F.Cu) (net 5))
 (segment (start 27.8 24.5675) (end 27.77 24.5975) (width 1.27) (layer F.Cu) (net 47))
 (segment (start 27.8 24.52) (end 27.8 24.5675) (width 1.27) (layer F.Cu) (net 47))
 (segment (start 27.77 24.5975) (end 27.77 27.12) (width 1.27) (layer F.Cu) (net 47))
 (segment (start 25.5 29.39) (end 22.86 29.39) (width 1.27) (layer F.Cu) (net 47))
 (segment (start 27.77 27.12) (end 25.5 29.39) (width 1.27) (layer F.Cu) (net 47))
 (segment (start 53.17134 61.08299) (end 46.97134 67.28299) (width 1.27) (layer F.Cu) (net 22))
 (segment (start 66.926579 61.08299) (end 53.17134 61.08299) (width 1.27) (layer F.Cu) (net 22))
 (segment (start 36.91 67.28299) (end 36.91 60.65567) (width 1.27) (layer F.Cu) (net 22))
 (segment (start 36.91 60.65567) (end 31.73299 55.47866) (width 1.27) (layer F.Cu) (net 22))
 (segment (start 46.97134 67.28299) (end 36.91 67.28299) (width 1.27) (layer F.Cu) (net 22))
 (segment (start 27.754229 45.440707) (end 31.683697 45.440707) (width 1.27) (layer F.Cu) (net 22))
 (segment (start 31.73299 45.49) (end 31.73299 55.47866) (width 1.27) (layer F.Cu) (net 22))
 (segment (start 31.683697 45.440707) (end 31.73299 45.49) (width 1.27) (layer F.Cu) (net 22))
 (segment (start 43.73 53.51) (end 40.23 50.01) (width 1.27) (layer F.Cu) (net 2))
 (segment (start 59.23 53.51) (end 43.73 53.51) (width 1.27) (layer F.Cu) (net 2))
 (segment (start 54.43701 69.34) (end 54.437009 65.548349) (width 1.27) (layer B.Cu) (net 2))
 (segment (start 54.437009 65.548349) (end 51.93165 63.04299) (width 1.27) (layer B.Cu) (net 2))
 (segment (start 51.93165 63.04299) (end 48.36299 63.04299) (width 1.27) (layer B.Cu) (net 2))
 (segment (start 40.23 54.91) (end 40.23 50.01) (width 1.27) (layer B.Cu) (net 2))
 (segment (start 48.36299 63.04299) (end 40.23 54.91) (width 1.27) (layer B.Cu) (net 2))
 (segment (start 67.74 41.22) (end 69.15 41.22) (width 1.27) (layer B.Cu) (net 33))
 (segment (start 67.24 40.72) (end 67.74 41.22) (width 1.27) (layer B.Cu) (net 33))
 (segment (start 31.179999 30.089999) (end 33.439999 30.089999) (width 1.27) (layer B.Cu) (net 33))
 (segment (start 33.439999 30.089999) (end 40.88 37.53) (width 1.27) (layer B.Cu) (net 33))
 (segment (start 67.24 38.85567) (end 67.24 40.72) (width 1.27) (layer B.Cu) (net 33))
 (segment (start 40.88 37.53) (end 65.91433 37.53) (width 1.27) (layer B.Cu) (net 33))
 (segment (start 30.48 29.39) (end 31.179999 30.089999) (width 1.27) (layer B.Cu) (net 33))
 (segment (start 65.91433 37.53) (end 67.24 38.85567) (width 1.27) (layer B.Cu) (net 33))
 (segment (start 63.17 28.52) (end 62.36 27.71) (width 1.27) (layer B.Cu) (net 41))
 (segment (start 69.15 28.52) (end 63.17 28.52) (width 1.27) (layer B.Cu) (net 41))
 (segment (start 63.17 25.98) (end 62.36 25.17) (width 1.27) (layer B.Cu) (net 42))
 (segment (start 69.15 25.98) (end 63.17 25.98) (width 1.27) (layer B.Cu) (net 42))
 (segment (start 53.04 66.12701) (end 53.04 71.45) (width 1.27) (layer B.Cu) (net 1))
 (segment (start 45.73 23.58) (end 43.92 25.39) (width 1.27) (layer B.Cu) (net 4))
 (segment (start 45.73 21.41) (end 45.73 23.58) (width 1.27) (layer B.Cu) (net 4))
 (segment (start 37.47 22.732792) (end 37.47 21.46) (width 1.27) (layer B.Cu) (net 4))
 (segment (start 40.127208 25.39) (end 37.47 22.732792) (width 1.27) (layer B.Cu) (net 4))
 (segment (start 43.92 25.39) (end 40.127208 25.39) (width 1.27) (layer B.Cu) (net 4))
 (segment (start 26.07 21.49) (end 31.52 21.49) (width 1.27) (layer F.Cu) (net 3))
 (segment (start 31.52 21.49) (end 34.31 24.28) (width 1.27) (layer F.Cu) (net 3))
 (segment (start 40.01 23.63) (end 40.01 21.46) (width 1.27) (layer F.Cu) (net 3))
 (segment (start 39.36 24.28) (end 40.01 23.63) (width 1.27) (layer F.Cu) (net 3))
 (segment (start 34.31 24.28) (end 39.36 24.28) (width 1.27) (layer F.Cu) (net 3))
 (segment (start 32.17567 26.85) (end 41.45866 36.13299) (width 1.27) (layer B.Cu) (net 40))
 (segment (start 27.754229 50.520707) (end 23.920707 50.520707) (width 1.27) (layer B.Cu) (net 40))
 (segment (start 28.09 26.85) (end 32.17567 26.85) (width 1.27) (layer B.Cu) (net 40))
 (segment (start 23.920707 50.520707) (end 23.920707 38.009293) (width 1.27) (layer B.Cu) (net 40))
 (segment (start 23.920707 38.009293) (end 27.05 34.88) (width 1.27) (layer B.Cu) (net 40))
 (segment (start 27.05 34.88) (end 27.05 27.89) (width 1.27) (layer B.Cu) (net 40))
 (segment (start 27.05 27.89) (end 28.09 26.85) (width 1.27) (layer B.Cu) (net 40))
 (segment (start 54.20701 36.13299) (end 53.16 36.13299) (width 1.27) (layer B.Cu) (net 40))
 (segment (start 60.09 30.25) (end 54.20701 36.13299) (width 1.27) (layer B.Cu) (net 40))
 (segment (start 62.36 30.25) (end 60.09 30.25) (width 1.27) (layer B.Cu) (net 40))
 (segment (start 41.45866 36.13299) (end 53.16 36.13299) (width 1.27) (layer B.Cu) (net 40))
 (segment (start 64.63 30.25) (end 62.36 30.25) (width 1.27) (layer B.Cu) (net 40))
 (segment (start 64.72567 30.15433) (end 64.63 30.25) (width 1.27) (layer B.Cu) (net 40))
 (segment (start 64.72567 29.92) (end 64.72567 30.15433) (width 1.27) (layer B.Cu) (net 40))
 (segment (start 43.19 28.74) (end 43.59 29.14) (width 1.27) (layer F.Cu) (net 5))
 (segment (start 43.19 21.41) (end 43.19 28.74) (width 1.27) (layer F.Cu) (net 5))
 (segment (start 34.90433 29.14) (end 43.59 29.14) (width 1.27) (layer F.Cu) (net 5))
 (segment (start 56.88299 20.83701) (end 73.16299 20.83701) (width 1.27) (layer F.Cu) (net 5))
 (segment (start 43.59 29.14) (end 48.58 29.14) (width 1.27) (layer F.Cu) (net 5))
 (segment (start 73.16299 20.83701) (end 73.16299 22.15) (width 1.27) (layer F.Cu) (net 5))
 (segment (start 48.58 29.14) (end 56.88299 20.83701) (width 1.27) (layer F.Cu) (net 5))
 (segment (start 30.272183 24.52) (end 29.88 24.912183) (width 1.27) (layer F.Cu) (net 46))
 (segment (start 30.34 24.52) (end 30.272183 24.52) (width 1.27) (layer F.Cu) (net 46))
 (segment (start 29.88 26.98567) (end 26.07866 30.78701) (width 1.27) (layer F.Cu) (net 46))
 (segment (start 26.07866 30.78701) (end 24.26299 30.78701) (width 1.27) (layer F.Cu) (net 46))
 (segment (start 23.11 31.94) (end 23.11 33.47) (width 1.27) (layer F.Cu) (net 46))
 (segment (start 24.26299 30.78701) (end 23.11 31.94) (width 1.27) (layer F.Cu) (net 46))
 (segment (start 30.34 26.79) (end 30.34 24.52) (width 1.27) (layer F.Cu) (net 46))
 (segment (start 30.14433 26.98567) (end 30.34 26.79) (width 1.27) (layer F.Cu) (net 46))
 (segment (start 29.88 26.98567) (end 30.14433 26.98567) (width 1.27) (layer F.Cu) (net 46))
 (segment (start 40.23 45.01) (end 40.23 38.85567) (width 1.27) (layer B.Cu) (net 2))
 (segment (start 34.84433 33.47) (end 30.73 33.47) (width 1.27) (layer B.Cu) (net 2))
 (segment (start 40.23 38.85567) (end 34.84433 33.47) (width 1.27) (layer B.Cu) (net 2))
 (segment (start 55.54 70.31863) (end 55.54 71.45) (width 1.27) (layer B.Cu) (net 2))
 (segment (start 54.56137 69.34) (end 55.54 70.31863) (width 1.27) (layer B.Cu) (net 2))
 (segment (start 54.43701 69.34) (end 54.56137 69.34) (width 1.27) (layer B.Cu) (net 2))
 (segment (start 55.54 72.58137) (end 55.54 71.45) (width 1.27) (layer F.Cu) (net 2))
 (segment (start 47.128398 71.36) (end 49.931388 74.16299) (width 1.27) (layer F.Cu) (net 2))
 (segment (start 53.95838 74.16299) (end 55.54 72.58137) (width 1.27) (layer F.Cu) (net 2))
 (segment (start 49.931388 74.16299) (end 53.95838 74.16299) (width 1.27) (layer F.Cu) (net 2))
 (segment (start 38.15 71.36) (end 47.128398 71.36) (width 1.27) (layer F.Cu) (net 2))
 (segment (start 47.869574 36.13299) (end 48.08 36.13299) (width 1.27) (layer F.Cu) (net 2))
 (segment (start 40.23 43.772564) (end 47.869574 36.13299) (width 1.27) (layer F.Cu) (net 2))
 (segment (start 40.23 45.01) (end 40.23 43.772564) (width 1.27) (layer F.Cu) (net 2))
 (segment (start 48.08 36.13299) (end 66.49299 36.13299) (width 1.27) (layer F.Cu) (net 2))
 (segment (start 65.842991 41.298661) (end 67.947919 43.403589) (width 1.27) (layer B.Cu) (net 6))
 (segment (start 65.84299 39.43433) (end 65.842991 41.298661) (width 1.27) (layer B.Cu) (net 6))
 (segment (start 59.23 55.51) (end 56.43 55.51) (width 1.27) (layer B.Cu) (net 6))
 (segment (start 56.43 42.088117) (end 56.42 42.078117) (width 1.27) (layer B.Cu) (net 6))
 (segment (start 56.43 55.51) (end 56.43 42.088117) (width 1.27) (layer B.Cu) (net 6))
 (segment (start 56.42 42.078117) (end 56.42 38.92701) (width 1.27) (layer B.Cu) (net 6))
 (segment (start 56.42 38.92701) (end 65.33567 38.92701) (width 1.27) (layer B.Cu) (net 6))
 (segment (start 65.33567 38.92701) (end 65.84299 39.43433) (width 1.27) (layer B.Cu) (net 6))
 (segment (start 68.793589 43.403589) (end 69.15 43.76) (width 1.27) (layer B.Cu) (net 6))
 (segment (start 67.947919 43.403589) (end 68.793589 43.403589) (width 1.27) (layer B.Cu) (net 6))
 (segment (start 67.03 23.44) (end 69.15 23.44) (width 1.27) (layer F.Cu) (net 44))
 (segment (start 64.63 30.5675) (end 64.63 25.84) (width 1.27) (layer F.Cu) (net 44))
 (segment (start 64.63 25.84) (end 67.03 23.44) (width 1.27) (layer F.Cu) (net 44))
 (segment (start 62.4075 32.79) (end 64.63 30.5675) (width 1.27) (layer F.Cu) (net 44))
 (segment (start 62.36 32.79) (end 62.4075 32.79) (width 1.27) (layer F.Cu) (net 44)))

